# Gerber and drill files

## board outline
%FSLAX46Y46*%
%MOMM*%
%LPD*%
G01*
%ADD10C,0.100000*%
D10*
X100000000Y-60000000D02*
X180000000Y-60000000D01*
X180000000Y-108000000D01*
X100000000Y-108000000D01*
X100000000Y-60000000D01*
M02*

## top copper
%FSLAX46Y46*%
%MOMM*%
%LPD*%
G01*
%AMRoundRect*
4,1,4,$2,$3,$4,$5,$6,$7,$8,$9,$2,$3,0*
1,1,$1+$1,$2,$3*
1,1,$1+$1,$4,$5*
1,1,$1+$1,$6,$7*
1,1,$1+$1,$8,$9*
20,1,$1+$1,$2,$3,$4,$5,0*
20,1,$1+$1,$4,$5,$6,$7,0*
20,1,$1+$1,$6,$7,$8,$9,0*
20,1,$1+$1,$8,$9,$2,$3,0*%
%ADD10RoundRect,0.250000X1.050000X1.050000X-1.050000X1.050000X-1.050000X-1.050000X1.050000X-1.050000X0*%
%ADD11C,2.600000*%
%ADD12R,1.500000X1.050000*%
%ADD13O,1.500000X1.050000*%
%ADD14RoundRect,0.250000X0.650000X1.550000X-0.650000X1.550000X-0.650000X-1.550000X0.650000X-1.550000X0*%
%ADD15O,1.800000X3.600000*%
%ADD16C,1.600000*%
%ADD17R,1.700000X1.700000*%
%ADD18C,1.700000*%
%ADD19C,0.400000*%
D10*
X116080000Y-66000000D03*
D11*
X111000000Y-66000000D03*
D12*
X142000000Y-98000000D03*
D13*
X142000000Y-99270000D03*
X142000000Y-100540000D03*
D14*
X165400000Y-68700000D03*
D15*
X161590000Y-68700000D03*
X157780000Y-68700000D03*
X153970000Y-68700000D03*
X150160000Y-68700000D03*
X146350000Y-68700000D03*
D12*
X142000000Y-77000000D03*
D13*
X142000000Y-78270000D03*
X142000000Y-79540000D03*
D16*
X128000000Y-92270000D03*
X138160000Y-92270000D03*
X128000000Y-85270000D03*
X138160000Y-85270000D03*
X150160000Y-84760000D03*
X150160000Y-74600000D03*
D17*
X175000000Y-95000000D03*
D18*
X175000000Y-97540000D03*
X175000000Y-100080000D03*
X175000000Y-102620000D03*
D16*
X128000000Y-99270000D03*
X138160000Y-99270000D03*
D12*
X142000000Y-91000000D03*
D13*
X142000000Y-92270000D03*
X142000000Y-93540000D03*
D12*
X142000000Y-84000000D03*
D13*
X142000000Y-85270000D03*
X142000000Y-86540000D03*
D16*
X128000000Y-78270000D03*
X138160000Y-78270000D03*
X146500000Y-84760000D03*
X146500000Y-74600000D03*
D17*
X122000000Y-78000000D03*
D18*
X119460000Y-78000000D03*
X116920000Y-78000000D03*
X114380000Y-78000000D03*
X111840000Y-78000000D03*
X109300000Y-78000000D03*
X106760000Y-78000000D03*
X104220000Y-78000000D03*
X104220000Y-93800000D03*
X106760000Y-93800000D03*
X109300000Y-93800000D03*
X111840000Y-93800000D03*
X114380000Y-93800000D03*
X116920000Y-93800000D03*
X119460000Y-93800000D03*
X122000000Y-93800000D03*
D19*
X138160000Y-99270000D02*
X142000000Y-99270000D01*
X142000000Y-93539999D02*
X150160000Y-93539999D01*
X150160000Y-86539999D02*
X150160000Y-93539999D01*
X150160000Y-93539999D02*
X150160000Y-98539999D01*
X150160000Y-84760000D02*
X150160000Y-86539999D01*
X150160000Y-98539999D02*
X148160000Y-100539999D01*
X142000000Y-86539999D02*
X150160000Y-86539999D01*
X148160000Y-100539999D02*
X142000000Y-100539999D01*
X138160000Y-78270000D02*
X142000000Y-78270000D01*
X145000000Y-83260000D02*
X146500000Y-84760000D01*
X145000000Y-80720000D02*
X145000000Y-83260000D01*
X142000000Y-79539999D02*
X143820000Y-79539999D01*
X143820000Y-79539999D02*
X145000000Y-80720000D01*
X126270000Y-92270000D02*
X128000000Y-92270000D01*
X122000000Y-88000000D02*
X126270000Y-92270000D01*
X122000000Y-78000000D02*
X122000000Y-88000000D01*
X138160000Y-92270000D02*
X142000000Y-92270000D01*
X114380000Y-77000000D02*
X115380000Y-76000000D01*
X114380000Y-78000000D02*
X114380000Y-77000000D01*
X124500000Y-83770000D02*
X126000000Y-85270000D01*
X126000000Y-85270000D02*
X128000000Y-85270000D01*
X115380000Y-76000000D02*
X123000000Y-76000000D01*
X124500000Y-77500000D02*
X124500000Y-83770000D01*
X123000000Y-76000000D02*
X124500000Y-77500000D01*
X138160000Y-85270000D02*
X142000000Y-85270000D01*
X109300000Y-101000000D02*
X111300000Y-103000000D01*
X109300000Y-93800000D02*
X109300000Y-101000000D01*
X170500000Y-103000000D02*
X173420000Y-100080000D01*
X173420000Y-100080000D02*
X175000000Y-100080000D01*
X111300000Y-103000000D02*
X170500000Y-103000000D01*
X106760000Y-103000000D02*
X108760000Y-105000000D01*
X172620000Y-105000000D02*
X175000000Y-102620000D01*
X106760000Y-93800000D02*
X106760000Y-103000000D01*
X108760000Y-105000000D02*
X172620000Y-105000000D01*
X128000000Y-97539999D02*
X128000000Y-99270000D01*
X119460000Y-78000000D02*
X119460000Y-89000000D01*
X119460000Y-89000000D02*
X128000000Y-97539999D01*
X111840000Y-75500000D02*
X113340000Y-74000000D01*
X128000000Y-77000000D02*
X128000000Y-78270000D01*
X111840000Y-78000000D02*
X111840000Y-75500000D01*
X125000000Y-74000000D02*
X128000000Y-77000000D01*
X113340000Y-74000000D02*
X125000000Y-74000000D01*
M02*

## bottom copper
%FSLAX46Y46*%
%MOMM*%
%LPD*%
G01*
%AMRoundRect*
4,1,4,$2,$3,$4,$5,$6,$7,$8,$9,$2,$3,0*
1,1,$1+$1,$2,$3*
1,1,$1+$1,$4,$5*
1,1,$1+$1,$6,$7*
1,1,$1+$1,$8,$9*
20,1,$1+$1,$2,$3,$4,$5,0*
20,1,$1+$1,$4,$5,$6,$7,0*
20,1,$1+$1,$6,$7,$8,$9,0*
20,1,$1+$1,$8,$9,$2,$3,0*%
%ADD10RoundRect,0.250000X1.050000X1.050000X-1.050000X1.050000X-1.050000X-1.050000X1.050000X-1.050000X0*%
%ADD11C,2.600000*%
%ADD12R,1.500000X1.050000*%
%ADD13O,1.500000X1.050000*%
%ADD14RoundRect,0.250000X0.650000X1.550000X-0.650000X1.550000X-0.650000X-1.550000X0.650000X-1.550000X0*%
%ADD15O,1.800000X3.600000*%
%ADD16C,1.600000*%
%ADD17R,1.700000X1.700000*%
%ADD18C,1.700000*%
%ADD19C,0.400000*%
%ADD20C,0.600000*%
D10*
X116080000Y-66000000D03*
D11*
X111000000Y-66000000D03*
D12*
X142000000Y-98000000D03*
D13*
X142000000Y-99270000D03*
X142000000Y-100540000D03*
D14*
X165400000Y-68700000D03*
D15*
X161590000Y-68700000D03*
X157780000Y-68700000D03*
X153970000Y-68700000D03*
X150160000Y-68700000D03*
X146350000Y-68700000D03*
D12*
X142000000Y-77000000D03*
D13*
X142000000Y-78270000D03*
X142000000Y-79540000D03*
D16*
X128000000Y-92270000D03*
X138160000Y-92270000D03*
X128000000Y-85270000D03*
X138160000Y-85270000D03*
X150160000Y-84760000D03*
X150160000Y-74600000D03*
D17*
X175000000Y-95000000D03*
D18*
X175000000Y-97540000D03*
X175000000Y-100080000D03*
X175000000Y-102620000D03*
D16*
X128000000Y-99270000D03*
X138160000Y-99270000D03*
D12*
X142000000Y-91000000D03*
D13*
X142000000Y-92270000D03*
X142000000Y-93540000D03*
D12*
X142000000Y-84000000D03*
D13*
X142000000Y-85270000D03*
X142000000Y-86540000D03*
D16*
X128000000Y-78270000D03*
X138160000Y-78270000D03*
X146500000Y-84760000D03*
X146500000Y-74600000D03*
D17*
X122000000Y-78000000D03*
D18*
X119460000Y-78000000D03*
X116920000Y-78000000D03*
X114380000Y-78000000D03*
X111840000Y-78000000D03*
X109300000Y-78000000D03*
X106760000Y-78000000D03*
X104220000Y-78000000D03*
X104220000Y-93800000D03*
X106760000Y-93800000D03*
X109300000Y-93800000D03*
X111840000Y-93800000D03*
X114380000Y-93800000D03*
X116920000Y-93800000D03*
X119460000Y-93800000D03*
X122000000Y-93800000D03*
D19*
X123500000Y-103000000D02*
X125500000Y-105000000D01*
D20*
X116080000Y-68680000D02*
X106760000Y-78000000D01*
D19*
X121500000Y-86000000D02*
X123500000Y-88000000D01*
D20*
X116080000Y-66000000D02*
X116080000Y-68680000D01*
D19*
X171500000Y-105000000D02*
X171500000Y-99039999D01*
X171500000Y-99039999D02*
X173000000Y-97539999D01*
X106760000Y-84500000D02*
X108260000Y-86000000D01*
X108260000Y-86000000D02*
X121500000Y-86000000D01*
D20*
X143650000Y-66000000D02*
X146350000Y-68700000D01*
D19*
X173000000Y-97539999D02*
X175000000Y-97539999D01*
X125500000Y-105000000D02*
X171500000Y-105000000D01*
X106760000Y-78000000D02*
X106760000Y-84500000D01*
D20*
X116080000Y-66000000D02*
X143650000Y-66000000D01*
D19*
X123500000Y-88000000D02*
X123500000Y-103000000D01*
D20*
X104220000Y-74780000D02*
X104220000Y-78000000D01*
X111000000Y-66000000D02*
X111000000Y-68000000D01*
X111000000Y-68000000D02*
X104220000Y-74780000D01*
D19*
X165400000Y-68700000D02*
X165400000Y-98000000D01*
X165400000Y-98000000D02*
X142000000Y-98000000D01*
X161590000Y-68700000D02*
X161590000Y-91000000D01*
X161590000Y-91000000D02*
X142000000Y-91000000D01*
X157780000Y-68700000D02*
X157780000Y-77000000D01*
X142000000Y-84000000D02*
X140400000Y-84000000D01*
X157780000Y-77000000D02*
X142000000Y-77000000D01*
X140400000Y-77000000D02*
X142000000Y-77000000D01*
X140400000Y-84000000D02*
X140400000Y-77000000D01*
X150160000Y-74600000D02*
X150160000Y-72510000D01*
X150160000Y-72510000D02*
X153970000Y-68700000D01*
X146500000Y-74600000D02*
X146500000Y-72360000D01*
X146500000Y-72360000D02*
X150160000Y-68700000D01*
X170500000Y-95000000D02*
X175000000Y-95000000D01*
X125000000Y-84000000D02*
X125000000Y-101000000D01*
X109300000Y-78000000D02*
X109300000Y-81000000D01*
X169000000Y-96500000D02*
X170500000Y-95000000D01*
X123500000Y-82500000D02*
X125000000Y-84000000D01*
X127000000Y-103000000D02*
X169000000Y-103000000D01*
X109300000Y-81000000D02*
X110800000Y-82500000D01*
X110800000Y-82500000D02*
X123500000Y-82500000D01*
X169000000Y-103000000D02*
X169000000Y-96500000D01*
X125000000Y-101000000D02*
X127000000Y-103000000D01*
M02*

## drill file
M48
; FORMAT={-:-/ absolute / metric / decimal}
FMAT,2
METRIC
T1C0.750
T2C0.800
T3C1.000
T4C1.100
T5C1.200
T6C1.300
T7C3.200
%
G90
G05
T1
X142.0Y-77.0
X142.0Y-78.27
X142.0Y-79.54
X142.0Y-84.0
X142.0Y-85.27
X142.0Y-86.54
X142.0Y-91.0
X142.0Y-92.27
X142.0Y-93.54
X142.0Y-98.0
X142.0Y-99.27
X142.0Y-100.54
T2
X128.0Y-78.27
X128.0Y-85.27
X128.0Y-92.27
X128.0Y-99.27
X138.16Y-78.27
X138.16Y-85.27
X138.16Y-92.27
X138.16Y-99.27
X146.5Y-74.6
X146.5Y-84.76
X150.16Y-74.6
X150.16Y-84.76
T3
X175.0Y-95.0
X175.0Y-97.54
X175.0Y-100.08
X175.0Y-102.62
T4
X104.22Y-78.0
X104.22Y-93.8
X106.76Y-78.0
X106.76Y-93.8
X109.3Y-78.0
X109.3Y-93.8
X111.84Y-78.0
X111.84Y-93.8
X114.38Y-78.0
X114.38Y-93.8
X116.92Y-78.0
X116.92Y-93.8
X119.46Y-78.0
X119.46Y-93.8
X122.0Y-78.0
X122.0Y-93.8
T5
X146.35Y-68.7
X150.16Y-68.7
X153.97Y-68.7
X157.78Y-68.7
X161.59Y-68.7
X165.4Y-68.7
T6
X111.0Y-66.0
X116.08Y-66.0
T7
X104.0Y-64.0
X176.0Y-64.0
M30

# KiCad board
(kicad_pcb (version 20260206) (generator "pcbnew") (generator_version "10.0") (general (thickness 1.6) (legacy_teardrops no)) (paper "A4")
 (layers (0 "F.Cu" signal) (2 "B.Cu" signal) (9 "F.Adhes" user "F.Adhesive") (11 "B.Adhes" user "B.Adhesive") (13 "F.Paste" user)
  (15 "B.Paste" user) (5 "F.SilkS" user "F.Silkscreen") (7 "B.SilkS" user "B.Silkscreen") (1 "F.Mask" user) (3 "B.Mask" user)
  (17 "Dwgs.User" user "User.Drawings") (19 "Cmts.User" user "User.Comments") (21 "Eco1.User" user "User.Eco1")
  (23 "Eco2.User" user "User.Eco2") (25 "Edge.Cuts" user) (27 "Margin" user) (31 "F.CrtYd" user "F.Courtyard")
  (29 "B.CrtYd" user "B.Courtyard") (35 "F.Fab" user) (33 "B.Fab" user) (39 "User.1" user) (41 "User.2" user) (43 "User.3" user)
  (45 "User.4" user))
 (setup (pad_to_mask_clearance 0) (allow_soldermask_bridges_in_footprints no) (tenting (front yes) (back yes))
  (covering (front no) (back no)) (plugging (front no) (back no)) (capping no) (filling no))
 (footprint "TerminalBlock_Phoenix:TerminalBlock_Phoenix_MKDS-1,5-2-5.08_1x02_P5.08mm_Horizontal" (layer "F.Cu") (at 116.08 66 180)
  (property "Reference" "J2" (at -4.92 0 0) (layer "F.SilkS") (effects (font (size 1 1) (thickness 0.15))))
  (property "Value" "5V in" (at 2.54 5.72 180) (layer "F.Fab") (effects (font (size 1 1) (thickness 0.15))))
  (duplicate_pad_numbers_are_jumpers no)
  (pad "1" thru_hole roundrect (at 0 0 180) (size 2.6 2.6) (drill 1.3) (layers "*.Cu" "*.Mask") (remove_unused_layers no)
   (roundrect_rratio 0.096154) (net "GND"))
  (pad "2" thru_hole circle (at 5.08 0 180) (size 2.6 2.6) (drill 1.3) (layers "*.Cu" "*.Mask") (remove_unused_layers no) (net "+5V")))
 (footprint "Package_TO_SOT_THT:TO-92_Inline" (layer "F.Cu") (at 142 98 -90)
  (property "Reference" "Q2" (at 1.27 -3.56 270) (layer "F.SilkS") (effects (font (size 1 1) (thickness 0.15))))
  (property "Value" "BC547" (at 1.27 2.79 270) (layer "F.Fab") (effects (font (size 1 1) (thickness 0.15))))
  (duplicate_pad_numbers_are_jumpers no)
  (pad "1" thru_hole rect (at 0 0 270) (size 1.05 1.5) (drill 0.75) (layers "*.Cu" "*.Mask") (remove_unused_layers no) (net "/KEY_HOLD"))
  (pad "2" thru_hole oval (at 1.27 0 270) (size 1.05 1.5) (drill 0.75) (layers "*.Cu" "*.Mask") (remove_unused_layers no) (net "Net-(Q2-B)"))
  (pad "3" thru_hole oval (at 2.54 0 270) (size 1.05 1.5) (drill 0.75) (layers "*.Cu" "*.Mask") (remove_unused_layers no) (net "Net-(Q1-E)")))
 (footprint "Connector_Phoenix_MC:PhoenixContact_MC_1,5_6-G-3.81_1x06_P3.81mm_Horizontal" (layer "F.Cu") (at 165.4 68.7 180)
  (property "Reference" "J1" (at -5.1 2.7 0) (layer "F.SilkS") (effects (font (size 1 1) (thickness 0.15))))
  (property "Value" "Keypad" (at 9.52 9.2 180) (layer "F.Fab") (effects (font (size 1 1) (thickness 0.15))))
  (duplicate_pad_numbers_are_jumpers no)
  (pad "1" thru_hole roundrect (at 0 0 180) (size 1.8 3.6) (drill 1.2) (layers "*.Cu" "*.Mask") (remove_unused_layers no)
   (roundrect_rratio 0.138889) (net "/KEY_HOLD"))
  (pad "2" thru_hole oval (at 3.81 0 180) (size 1.8 3.6) (drill 1.2) (layers "*.Cu" "*.Mask") (remove_unused_layers no) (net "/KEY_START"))
  (pad "3" thru_hole oval (at 7.62 0 180) (size 1.8 3.6) (drill 1.2) (layers "*.Cu" "*.Mask") (remove_unused_layers no)
   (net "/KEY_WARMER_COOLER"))
  (pad "4" thru_hole oval (at 11.43 0 180) (size 1.8 3.6) (drill 1.2) (layers "*.Cu" "*.Mask") (remove_unused_layers no) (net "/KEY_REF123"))
  (pad "5" thru_hole oval (at 15.24 0 180) (size 1.8 3.6) (drill 1.2) (layers "*.Cu" "*.Mask") (remove_unused_layers no) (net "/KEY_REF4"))
  (pad "6" thru_hole oval (at 19.05 0 180) (size 1.8 3.6) (drill 1.2) (layers "*.Cu" "*.Mask") (remove_unused_layers no) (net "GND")))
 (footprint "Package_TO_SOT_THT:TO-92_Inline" (layer "F.Cu") (at 142 77 -90)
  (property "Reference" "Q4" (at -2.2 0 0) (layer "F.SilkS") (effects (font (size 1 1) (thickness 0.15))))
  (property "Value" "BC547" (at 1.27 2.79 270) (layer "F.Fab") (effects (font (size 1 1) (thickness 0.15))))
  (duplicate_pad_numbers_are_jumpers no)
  (pad "1" thru_hole rect (at 0 0 270) (size 1.05 1.5) (drill 0.75) (layers "*.Cu" "*.Mask") (remove_unused_layers no)
   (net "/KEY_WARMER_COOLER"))
  (pad "2" thru_hole oval (at 1.27 0 270) (size 1.05 1.5) (drill 0.75) (layers "*.Cu" "*.Mask") (remove_unused_layers no) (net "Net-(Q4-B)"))
  (pad "3" thru_hole oval (at 2.54 0 270) (size 1.05 1.5) (drill 0.75) (layers "*.Cu" "*.Mask") (remove_unused_layers no) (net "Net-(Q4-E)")))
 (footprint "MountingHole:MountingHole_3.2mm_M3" (layer "F.Cu") (at 104 64)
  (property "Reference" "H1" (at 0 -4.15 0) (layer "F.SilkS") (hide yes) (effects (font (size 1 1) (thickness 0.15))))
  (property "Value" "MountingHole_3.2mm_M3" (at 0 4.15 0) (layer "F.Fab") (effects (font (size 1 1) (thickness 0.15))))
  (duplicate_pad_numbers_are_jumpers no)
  (pad "" np_thru_hole circle (at 0 0) (size 3.2 3.2) (drill 3.2) (layers "*.Cu" "*.Mask")))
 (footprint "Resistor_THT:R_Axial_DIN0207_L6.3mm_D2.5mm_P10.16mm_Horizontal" (layer "F.Cu") (at 128 92.27)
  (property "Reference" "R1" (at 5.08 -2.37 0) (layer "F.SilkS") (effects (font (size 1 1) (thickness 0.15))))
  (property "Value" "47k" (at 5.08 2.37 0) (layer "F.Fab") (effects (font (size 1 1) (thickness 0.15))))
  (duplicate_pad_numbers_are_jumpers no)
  (pad "1" thru_hole circle (at 0 0) (size 1.6 1.6) (drill 0.8) (layers "*.Cu" "*.Mask") (remove_unused_layers no) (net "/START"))
  (pad "2" thru_hole circle (at 10.16 0) (size 1.6 1.6) (drill 0.8) (layers "*.Cu" "*.Mask") (remove_unused_layers no) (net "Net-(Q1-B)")))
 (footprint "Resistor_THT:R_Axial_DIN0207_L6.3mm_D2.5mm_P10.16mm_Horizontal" (layer "F.Cu") (at 128 85.27)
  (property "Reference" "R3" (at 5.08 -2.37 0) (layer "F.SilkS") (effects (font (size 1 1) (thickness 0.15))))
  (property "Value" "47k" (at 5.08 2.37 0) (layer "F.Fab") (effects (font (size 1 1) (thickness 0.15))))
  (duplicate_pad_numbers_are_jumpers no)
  (pad "1" thru_hole circle (at 0 0) (size 1.6 1.6) (drill 0.8) (layers "*.Cu" "*.Mask") (remove_unused_layers no) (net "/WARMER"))
  (pad "2" thru_hole circle (at 10.16 0) (size 1.6 1.6) (drill 0.8) (layers "*.Cu" "*.Mask") (remove_unused_layers no) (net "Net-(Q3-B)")))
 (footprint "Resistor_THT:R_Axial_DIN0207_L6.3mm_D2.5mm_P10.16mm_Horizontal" (layer "F.Cu") (at 150.16 84.76 90)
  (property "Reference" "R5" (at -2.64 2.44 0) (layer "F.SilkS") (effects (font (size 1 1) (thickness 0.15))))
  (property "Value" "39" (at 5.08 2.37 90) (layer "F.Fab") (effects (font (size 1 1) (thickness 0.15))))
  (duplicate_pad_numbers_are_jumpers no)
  (pad "1" thru_hole circle (at 0 0 90) (size 1.6 1.6) (drill 0.8) (layers "*.Cu" "*.Mask") (remove_unused_layers no) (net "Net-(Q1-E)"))
  (pad "2" thru_hole circle (at 10.16 0 90) (size 1.6 1.6) (drill 0.8) (layers "*.Cu" "*.Mask") (remove_unused_layers no)
   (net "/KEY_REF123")))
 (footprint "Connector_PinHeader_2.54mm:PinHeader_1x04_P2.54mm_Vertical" (layer "F.Cu") (at 175 95)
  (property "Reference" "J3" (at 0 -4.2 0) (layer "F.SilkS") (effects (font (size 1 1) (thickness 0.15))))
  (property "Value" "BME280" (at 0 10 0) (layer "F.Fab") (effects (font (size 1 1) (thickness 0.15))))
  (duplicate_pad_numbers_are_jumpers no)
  (pad "1" thru_hole rect (at 0 0) (size 1.7 1.7) (drill 1) (layers "*.Cu" "*.Mask") (remove_unused_layers no) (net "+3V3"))
  (pad "2" thru_hole circle (at 0 2.54) (size 1.7 1.7) (drill 1) (layers "*.Cu" "*.Mask") (remove_unused_layers no) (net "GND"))
  (pad "3" thru_hole circle (at 0 5.08) (size 1.7 1.7) (drill 1) (layers "*.Cu" "*.Mask") (remove_unused_layers no) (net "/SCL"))
  (pad "4" thru_hole circle (at 0 7.62) (size 1.7 1.7) (drill 1) (layers "*.Cu" "*.Mask") (remove_unused_layers no) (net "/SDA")))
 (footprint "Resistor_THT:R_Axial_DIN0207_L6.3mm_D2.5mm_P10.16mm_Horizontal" (layer "F.Cu") (at 128 99.27)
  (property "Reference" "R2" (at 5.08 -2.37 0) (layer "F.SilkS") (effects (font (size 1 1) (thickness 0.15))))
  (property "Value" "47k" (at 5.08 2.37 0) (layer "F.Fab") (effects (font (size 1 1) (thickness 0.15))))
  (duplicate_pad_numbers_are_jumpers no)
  (pad "1" thru_hole circle (at 0 0) (size 1.6 1.6) (drill 0.8) (layers "*.Cu" "*.Mask") (remove_unused_layers no) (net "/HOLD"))
  (pad "2" thru_hole circle (at 10.16 0) (size 1.6 1.6) (drill 0.8) (layers "*.Cu" "*.Mask") (remove_unused_layers no) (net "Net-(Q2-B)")))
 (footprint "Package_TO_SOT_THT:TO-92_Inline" (layer "F.Cu") (at 142 91 -90)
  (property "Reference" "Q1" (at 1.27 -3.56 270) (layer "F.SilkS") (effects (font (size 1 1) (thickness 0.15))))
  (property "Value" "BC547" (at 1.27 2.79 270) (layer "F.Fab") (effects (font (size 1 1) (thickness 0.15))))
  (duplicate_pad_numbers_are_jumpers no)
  (pad "1" thru_hole rect (at 0 0 270) (size 1.05 1.5) (drill 0.75) (layers "*.Cu" "*.Mask") (remove_unused_layers no) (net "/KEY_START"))
  (pad "2" thru_hole oval (at 1.27 0 270) (size 1.05 1.5) (drill 0.75) (layers "*.Cu" "*.Mask") (remove_unused_layers no) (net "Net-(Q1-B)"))
  (pad "3" thru_hole oval (at 2.54 0 270) (size 1.05 1.5) (drill 0.75) (layers "*.Cu" "*.Mask") (remove_unused_layers no) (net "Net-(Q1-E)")))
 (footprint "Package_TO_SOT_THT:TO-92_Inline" (layer "F.Cu") (at 142 84 -90)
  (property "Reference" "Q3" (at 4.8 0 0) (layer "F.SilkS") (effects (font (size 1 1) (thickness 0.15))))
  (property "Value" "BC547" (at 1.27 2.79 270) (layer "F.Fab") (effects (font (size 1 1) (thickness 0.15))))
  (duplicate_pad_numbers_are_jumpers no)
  (pad "1" thru_hole rect (at 0 0 270) (size 1.05 1.5) (drill 0.75) (layers "*.Cu" "*.Mask") (remove_unused_layers no)
   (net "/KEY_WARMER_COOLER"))
  (pad "2" thru_hole oval (at 1.27 0 270) (size 1.05 1.5) (drill 0.75) (layers "*.Cu" "*.Mask") (remove_unused_layers no) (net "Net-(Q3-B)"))
  (pad "3" thru_hole oval (at 2.54 0 270) (size 1.05 1.5) (drill 0.75) (layers "*.Cu" "*.Mask") (remove_unused_layers no) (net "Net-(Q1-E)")))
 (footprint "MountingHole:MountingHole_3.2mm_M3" (layer "F.Cu") (at 176 64)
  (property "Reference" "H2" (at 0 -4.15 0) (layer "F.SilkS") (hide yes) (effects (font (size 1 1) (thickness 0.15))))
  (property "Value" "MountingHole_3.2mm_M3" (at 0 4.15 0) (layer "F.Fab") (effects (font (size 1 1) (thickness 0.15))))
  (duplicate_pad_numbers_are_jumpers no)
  (pad "" np_thru_hole circle (at 0 0) (size 3.2 3.2) (drill 3.2) (layers "*.Cu" "*.Mask")))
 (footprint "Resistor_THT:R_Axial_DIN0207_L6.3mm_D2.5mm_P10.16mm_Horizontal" (layer "F.Cu") (at 128 78.27)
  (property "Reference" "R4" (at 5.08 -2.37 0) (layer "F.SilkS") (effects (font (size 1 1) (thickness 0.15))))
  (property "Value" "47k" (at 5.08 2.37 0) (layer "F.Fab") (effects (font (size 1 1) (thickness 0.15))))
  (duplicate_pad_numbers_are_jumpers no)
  (pad "1" thru_hole circle (at 0 0) (size 1.6 1.6) (drill 0.8) (layers "*.Cu" "*.Mask") (remove_unused_layers no) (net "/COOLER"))
  (pad "2" thru_hole circle (at 10.16 0) (size 1.6 1.6) (drill 0.8) (layers "*.Cu" "*.Mask") (remove_unused_layers no) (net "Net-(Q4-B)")))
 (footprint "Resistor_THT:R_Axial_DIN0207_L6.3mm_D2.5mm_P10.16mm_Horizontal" (layer "F.Cu") (at 146.5 84.76 90)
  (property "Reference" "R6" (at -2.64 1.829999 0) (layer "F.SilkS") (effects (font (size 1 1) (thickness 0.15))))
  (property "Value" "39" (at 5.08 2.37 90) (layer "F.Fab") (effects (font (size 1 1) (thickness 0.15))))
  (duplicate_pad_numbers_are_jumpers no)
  (pad "1" thru_hole circle (at 0 0 90) (size 1.6 1.6) (drill 0.8) (layers "*.Cu" "*.Mask") (remove_unused_layers no) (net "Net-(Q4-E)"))
  (pad "2" thru_hole circle (at 10.16 0 90) (size 1.6 1.6) (drill 0.8) (layers "*.Cu" "*.Mask") (remove_unused_layers no) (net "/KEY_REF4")))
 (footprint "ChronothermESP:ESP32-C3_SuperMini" (layer "F.Cu") (at 122 78 -90)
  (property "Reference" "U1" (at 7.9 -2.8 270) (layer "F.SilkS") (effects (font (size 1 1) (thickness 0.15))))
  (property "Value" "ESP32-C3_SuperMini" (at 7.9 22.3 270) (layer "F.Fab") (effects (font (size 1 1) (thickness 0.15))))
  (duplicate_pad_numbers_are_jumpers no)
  (pad "1" thru_hole rect (at 0 0 270) (size 1.7 1.7) (drill 1.1) (layers "*.Cu" "*.Mask") (remove_unused_layers no) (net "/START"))
  (pad "2" thru_hole circle (at 0 2.54 270) (size 1.7 1.7) (drill 1.1) (layers "*.Cu" "*.Mask") (remove_unused_layers no) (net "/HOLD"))
  (pad "3" thru_hole circle (at 0 5.08 270) (size 1.7 1.7) (drill 1.1) (layers "*.Cu" "*.Mask") (remove_unused_layers no)
   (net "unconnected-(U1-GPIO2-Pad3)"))
  (pad "4" thru_hole circle (at 0 7.62 270) (size 1.7 1.7) (drill 1.1) (layers "*.Cu" "*.Mask") (remove_unused_layers no) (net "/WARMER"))
  (pad "5" thru_hole circle (at 0 10.16 270) (size 1.7 1.7) (drill 1.1) (layers "*.Cu" "*.Mask") (remove_unused_layers no) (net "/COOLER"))
  (pad "6" thru_hole circle (at 0 12.7 270) (size 1.7 1.7) (drill 1.1) (layers "*.Cu" "*.Mask") (remove_unused_layers no) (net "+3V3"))
  (pad "7" thru_hole circle (at 0 15.24 270) (size 1.7 1.7) (drill 1.1) (layers "*.Cu" "*.Mask") (remove_unused_layers no) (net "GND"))
  (pad "8" thru_hole circle (at 0 17.78 270) (size 1.7 1.7) (drill 1.1) (layers "*.Cu" "*.Mask") (remove_unused_layers no) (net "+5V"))
  (pad "9" thru_hole circle (at 15.8 17.78 270) (size 1.7 1.7) (drill 1.1) (layers "*.Cu" "*.Mask") (remove_unused_layers no)
   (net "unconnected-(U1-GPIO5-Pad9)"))
  (pad "10" thru_hole circle (at 15.8 15.24 270) (size 1.7 1.7) (drill 1.1) (layers "*.Cu" "*.Mask") (remove_unused_layers no) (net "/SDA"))
  (pad "11" thru_hole circle (at 15.8 12.7 270) (size 1.7 1.7) (drill 1.1) (layers "*.Cu" "*.Mask") (remove_unused_layers no) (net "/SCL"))
  (pad "12" thru_hole circle (at 15.8 10.16 270) (size 1.7 1.7) (drill 1.1) (layers "*.Cu" "*.Mask") (remove_unused_layers no)
   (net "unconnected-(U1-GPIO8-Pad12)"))
  (pad "13" thru_hole circle (at 15.8 7.62 270) (size 1.7 1.7) (drill 1.1) (layers "*.Cu" "*.Mask") (remove_unused_layers no)
   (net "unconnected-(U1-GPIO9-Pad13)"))
  (pad "14" thru_hole circle (at 15.8 5.08 270) (size 1.7 1.7) (drill 1.1) (layers "*.Cu" "*.Mask") (remove_unused_layers no)
   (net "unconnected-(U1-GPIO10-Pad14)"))
  (pad "15" thru_hole circle (at 15.8 2.54 270) (size 1.7 1.7) (drill 1.1) (layers "*.Cu" "*.Mask") (remove_unused_layers no)
   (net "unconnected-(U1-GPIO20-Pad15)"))
  (pad "16" thru_hole circle (at 15.8 0 270) (size 1.7 1.7) (drill 1.1) (layers "*.Cu" "*.Mask") (remove_unused_layers no)
   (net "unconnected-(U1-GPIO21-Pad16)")))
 (gr_rect (start 100 60) (end 180 108) (stroke (width 0.1) (type default)) (fill no) (layer "Edge.Cuts"))
 (segment (start 123.5 103) (end 125.5 105) (width 0.4) (layer "B.Cu") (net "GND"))
 (segment (start 116.08 68.68) (end 106.76 78) (width 0.6) (layer "B.Cu") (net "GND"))
 (segment (start 121.5 86) (end 123.5 88) (width 0.4) (layer "B.Cu") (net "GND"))
 (segment (start 116.08 66) (end 116.08 68.68) (width 0.6) (layer "B.Cu") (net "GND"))
 (segment (start 171.5 105) (end 171.5 99.039999) (width 0.4) (layer "B.Cu") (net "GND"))
 (segment (start 171.5 99.039999) (end 173 97.539999) (width 0.4) (layer "B.Cu") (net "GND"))
 (segment (start 106.76 84.5) (end 108.26 86) (width 0.4) (layer "B.Cu") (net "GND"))
 (segment (start 108.26 86) (end 121.5 86) (width 0.4) (layer "B.Cu") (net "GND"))
 (segment (start 143.65 66) (end 146.35 68.7) (width 0.6) (layer "B.Cu") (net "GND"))
 (segment (start 173 97.539999) (end 175 97.539999) (width 0.4) (layer "B.Cu") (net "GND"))
 (segment (start 125.5 105) (end 171.5 105) (width 0.4) (layer "B.Cu") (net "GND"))
 (segment (start 106.76 78) (end 106.76 84.5) (width 0.4) (layer "B.Cu") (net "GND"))
 (segment (start 116.08 66) (end 143.65 66) (width 0.6) (layer "B.Cu") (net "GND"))
 (segment (start 123.5 88) (end 123.5 103) (width 0.4) (layer "B.Cu") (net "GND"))
 (segment (start 104.22 74.78) (end 104.22 78) (width 0.6) (layer "B.Cu") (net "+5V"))
 (segment (start 111 66) (end 111 68) (width 0.6) (layer "B.Cu") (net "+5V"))
 (segment (start 111 68) (end 104.22 74.78) (width 0.6) (layer "B.Cu") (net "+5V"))
 (segment (start 165.4 68.7) (end 165.4 98) (width 0.4) (layer "B.Cu") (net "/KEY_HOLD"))
 (segment (start 165.4 98) (end 142 98) (width 0.4) (layer "B.Cu") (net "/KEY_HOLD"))
 (segment (start 138.16 99.27) (end 142 99.27) (width 0.4) (layer "F.Cu") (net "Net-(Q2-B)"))
 (segment (start 142 93.539999) (end 150.16 93.539999) (width 0.4) (layer "F.Cu") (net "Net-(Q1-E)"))
 (segment (start 150.16 86.539999) (end 150.16 93.539999) (width 0.4) (layer "F.Cu") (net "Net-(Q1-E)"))
 (segment (start 150.16 93.539999) (end 150.16 98.539999) (width 0.4) (layer "F.Cu") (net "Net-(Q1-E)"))
 (segment (start 150.16 84.76) (end 150.16 86.539999) (width 0.4) (layer "F.Cu") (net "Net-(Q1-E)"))
 (segment (start 150.16 98.539999) (end 148.16 100.539999) (width 0.4) (layer "F.Cu") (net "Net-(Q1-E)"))
 (segment (start 142 86.539999) (end 150.16 86.539999) (width 0.4) (layer "F.Cu") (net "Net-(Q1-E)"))
 (segment (start 148.16 100.539999) (end 142 100.539999) (width 0.4) (layer "F.Cu") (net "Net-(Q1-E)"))
 (segment (start 161.59 68.7) (end 161.59 91) (width 0.4) (layer "B.Cu") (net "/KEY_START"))
 (segment (start 161.59 91) (end 142 91) (width 0.4) (layer "B.Cu") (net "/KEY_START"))
 (segment (start 157.78 68.7) (end 157.78 77) (width 0.4) (layer "B.Cu") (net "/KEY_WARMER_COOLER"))
 (segment (start 142 84) (end 140.4 84) (width 0.4) (layer "B.Cu") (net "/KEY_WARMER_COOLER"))
 (segment (start 157.78 77) (end 142 77) (width 0.4) (layer "B.Cu") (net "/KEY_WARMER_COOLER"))
 (segment (start 140.4 77) (end 142 77) (width 0.4) (layer "B.Cu") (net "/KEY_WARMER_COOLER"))
 (segment (start 140.4 84) (end 140.4 77) (width 0.4) (layer "B.Cu") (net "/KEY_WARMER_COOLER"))
 (segment (start 150.16 74.6) (end 150.16 72.51) (width 0.4) (layer "B.Cu") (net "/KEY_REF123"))
 (segment (start 150.16 72.51) (end 153.97 68.7) (width 0.4) (layer "B.Cu") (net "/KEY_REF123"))
 (segment (start 146.5 74.6) (end 146.5 72.36) (width 0.4) (layer "B.Cu") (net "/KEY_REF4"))
 (segment (start 146.5 72.36) (end 150.16 68.7) (width 0.4) (layer "B.Cu") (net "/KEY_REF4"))
 (segment (start 138.16 78.27) (end 142 78.27) (width 0.4) (layer "F.Cu") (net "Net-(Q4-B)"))
 (segment (start 145 83.26) (end 146.5 84.76) (width 0.4) (layer "F.Cu") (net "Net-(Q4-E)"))
 (segment (start 145 80.72) (end 145 83.26) (width 0.4) (layer "F.Cu") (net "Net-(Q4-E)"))
 (segment (start 142 79.539999) (end 143.82 79.539999) (width 0.4) (layer "F.Cu") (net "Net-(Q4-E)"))
 (segment (start 143.82 79.539999) (end 145 80.72) (width 0.4) (layer "F.Cu") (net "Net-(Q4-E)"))
 (segment (start 126.27 92.27) (end 128 92.27) (width 0.4) (layer "F.Cu") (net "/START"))
 (segment (start 122 88) (end 126.27 92.27) (width 0.4) (layer "F.Cu") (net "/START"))
 (segment (start 122 78) (end 122 88) (width 0.4) (layer "F.Cu") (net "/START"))
 (segment (start 138.16 92.27) (end 142 92.27) (width 0.4) (layer "F.Cu") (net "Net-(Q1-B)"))
 (segment (start 114.38 77) (end 115.38 76) (width 0.4) (layer "F.Cu") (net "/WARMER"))
 (segment (start 114.38 78) (end 114.38 77) (width 0.4) (layer "F.Cu") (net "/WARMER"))
 (segment (start 124.5 83.77) (end 126 85.27) (width 0.4) (layer "F.Cu") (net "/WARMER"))
 (segment (start 126 85.27) (end 128 85.27) (width 0.4) (layer "F.Cu") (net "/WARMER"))
 (segment (start 115.38 76) (end 123 76) (width 0.4) (layer "F.Cu") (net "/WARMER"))
 (segment (start 124.5 77.5) (end 124.5 83.77) (width 0.4) (layer "F.Cu") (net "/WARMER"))
 (segment (start 123 76) (end 124.5 77.5) (width 0.4) (layer "F.Cu") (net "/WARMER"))
 (segment (start 138.16 85.27) (end 142 85.27) (width 0.4) (layer "F.Cu") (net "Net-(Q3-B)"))
 (segment (start 170.5 95) (end 175 95) (width 0.4) (layer "B.Cu") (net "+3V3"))
 (segment (start 125 84) (end 125 101) (width 0.4) (layer "B.Cu") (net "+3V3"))
 (segment (start 109.3 78) (end 109.3 81) (width 0.4) (layer "B.Cu") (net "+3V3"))
 (segment (start 169 96.5) (end 170.5 95) (width 0.4) (layer "B.Cu") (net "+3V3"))
 (segment (start 123.5 82.5) (end 125 84) (width 0.4) (layer "B.Cu") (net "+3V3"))
 (segment (start 127 103) (end 169 103) (width 0.4) (layer "B.Cu") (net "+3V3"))
 (segment (start 109.3 81) (end 110.8 82.5) (width 0.4) (layer "B.Cu") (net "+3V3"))
 (segment (start 110.8 82.5) (end 123.5 82.5) (width 0.4) (layer "B.Cu") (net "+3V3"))
 (segment (start 169 103) (end 169 96.5) (width 0.4) (layer "B.Cu") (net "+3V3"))
 (segment (start 125 101) (end 127 103) (width 0.4) (layer "B.Cu") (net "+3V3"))
 (segment (start 109.3 101) (end 111.3 103) (width 0.4) (layer "F.Cu") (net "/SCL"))
 (segment (start 109.3 93.8) (end 109.3 101) (width 0.4) (layer "F.Cu") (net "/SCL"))
 (segment (start 170.5 103) (end 173.42 100.08) (width 0.4) (layer "F.Cu") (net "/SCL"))
 (segment (start 173.42 100.08) (end 175 100.08) (width 0.4) (layer "F.Cu") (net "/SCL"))
 (segment (start 111.3 103) (end 170.5 103) (width 0.4) (layer "F.Cu") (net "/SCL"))
 (segment (start 106.76 103) (end 108.76 105) (width 0.4) (layer "F.Cu") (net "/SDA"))
 (segment (start 172.62 105) (end 175 102.62) (width 0.4) (layer "F.Cu") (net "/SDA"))
 (segment (start 106.76 93.8) (end 106.76 103) (width 0.4) (layer "F.Cu") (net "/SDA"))
 (segment (start 108.76 105) (end 172.62 105) (width 0.4) (layer "F.Cu") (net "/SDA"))
 (segment (start 128 97.539999) (end 128 99.27) (width 0.4) (layer "F.Cu") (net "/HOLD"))
 (segment (start 119.46 78) (end 119.46 89) (width 0.4) (layer "F.Cu") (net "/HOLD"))
 (segment (start 119.46 89) (end 128 97.539999) (width 0.4) (layer "F.Cu") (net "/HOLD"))
 (segment (start 111.84 75.5) (end 113.34 74) (width 0.4) (layer "F.Cu") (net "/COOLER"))
 (segment (start 128 77) (end 128 78.27) (width 0.4) (layer "F.Cu") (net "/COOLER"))
 (segment (start 111.84 78) (end 111.84 75.5) (width 0.4) (layer "F.Cu") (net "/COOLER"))
 (segment (start 125 74) (end 128 77) (width 0.4) (layer "F.Cu") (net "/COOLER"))
 (segment (start 113.34 74) (end 125 74) (width 0.4) (layer "F.Cu") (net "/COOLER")))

